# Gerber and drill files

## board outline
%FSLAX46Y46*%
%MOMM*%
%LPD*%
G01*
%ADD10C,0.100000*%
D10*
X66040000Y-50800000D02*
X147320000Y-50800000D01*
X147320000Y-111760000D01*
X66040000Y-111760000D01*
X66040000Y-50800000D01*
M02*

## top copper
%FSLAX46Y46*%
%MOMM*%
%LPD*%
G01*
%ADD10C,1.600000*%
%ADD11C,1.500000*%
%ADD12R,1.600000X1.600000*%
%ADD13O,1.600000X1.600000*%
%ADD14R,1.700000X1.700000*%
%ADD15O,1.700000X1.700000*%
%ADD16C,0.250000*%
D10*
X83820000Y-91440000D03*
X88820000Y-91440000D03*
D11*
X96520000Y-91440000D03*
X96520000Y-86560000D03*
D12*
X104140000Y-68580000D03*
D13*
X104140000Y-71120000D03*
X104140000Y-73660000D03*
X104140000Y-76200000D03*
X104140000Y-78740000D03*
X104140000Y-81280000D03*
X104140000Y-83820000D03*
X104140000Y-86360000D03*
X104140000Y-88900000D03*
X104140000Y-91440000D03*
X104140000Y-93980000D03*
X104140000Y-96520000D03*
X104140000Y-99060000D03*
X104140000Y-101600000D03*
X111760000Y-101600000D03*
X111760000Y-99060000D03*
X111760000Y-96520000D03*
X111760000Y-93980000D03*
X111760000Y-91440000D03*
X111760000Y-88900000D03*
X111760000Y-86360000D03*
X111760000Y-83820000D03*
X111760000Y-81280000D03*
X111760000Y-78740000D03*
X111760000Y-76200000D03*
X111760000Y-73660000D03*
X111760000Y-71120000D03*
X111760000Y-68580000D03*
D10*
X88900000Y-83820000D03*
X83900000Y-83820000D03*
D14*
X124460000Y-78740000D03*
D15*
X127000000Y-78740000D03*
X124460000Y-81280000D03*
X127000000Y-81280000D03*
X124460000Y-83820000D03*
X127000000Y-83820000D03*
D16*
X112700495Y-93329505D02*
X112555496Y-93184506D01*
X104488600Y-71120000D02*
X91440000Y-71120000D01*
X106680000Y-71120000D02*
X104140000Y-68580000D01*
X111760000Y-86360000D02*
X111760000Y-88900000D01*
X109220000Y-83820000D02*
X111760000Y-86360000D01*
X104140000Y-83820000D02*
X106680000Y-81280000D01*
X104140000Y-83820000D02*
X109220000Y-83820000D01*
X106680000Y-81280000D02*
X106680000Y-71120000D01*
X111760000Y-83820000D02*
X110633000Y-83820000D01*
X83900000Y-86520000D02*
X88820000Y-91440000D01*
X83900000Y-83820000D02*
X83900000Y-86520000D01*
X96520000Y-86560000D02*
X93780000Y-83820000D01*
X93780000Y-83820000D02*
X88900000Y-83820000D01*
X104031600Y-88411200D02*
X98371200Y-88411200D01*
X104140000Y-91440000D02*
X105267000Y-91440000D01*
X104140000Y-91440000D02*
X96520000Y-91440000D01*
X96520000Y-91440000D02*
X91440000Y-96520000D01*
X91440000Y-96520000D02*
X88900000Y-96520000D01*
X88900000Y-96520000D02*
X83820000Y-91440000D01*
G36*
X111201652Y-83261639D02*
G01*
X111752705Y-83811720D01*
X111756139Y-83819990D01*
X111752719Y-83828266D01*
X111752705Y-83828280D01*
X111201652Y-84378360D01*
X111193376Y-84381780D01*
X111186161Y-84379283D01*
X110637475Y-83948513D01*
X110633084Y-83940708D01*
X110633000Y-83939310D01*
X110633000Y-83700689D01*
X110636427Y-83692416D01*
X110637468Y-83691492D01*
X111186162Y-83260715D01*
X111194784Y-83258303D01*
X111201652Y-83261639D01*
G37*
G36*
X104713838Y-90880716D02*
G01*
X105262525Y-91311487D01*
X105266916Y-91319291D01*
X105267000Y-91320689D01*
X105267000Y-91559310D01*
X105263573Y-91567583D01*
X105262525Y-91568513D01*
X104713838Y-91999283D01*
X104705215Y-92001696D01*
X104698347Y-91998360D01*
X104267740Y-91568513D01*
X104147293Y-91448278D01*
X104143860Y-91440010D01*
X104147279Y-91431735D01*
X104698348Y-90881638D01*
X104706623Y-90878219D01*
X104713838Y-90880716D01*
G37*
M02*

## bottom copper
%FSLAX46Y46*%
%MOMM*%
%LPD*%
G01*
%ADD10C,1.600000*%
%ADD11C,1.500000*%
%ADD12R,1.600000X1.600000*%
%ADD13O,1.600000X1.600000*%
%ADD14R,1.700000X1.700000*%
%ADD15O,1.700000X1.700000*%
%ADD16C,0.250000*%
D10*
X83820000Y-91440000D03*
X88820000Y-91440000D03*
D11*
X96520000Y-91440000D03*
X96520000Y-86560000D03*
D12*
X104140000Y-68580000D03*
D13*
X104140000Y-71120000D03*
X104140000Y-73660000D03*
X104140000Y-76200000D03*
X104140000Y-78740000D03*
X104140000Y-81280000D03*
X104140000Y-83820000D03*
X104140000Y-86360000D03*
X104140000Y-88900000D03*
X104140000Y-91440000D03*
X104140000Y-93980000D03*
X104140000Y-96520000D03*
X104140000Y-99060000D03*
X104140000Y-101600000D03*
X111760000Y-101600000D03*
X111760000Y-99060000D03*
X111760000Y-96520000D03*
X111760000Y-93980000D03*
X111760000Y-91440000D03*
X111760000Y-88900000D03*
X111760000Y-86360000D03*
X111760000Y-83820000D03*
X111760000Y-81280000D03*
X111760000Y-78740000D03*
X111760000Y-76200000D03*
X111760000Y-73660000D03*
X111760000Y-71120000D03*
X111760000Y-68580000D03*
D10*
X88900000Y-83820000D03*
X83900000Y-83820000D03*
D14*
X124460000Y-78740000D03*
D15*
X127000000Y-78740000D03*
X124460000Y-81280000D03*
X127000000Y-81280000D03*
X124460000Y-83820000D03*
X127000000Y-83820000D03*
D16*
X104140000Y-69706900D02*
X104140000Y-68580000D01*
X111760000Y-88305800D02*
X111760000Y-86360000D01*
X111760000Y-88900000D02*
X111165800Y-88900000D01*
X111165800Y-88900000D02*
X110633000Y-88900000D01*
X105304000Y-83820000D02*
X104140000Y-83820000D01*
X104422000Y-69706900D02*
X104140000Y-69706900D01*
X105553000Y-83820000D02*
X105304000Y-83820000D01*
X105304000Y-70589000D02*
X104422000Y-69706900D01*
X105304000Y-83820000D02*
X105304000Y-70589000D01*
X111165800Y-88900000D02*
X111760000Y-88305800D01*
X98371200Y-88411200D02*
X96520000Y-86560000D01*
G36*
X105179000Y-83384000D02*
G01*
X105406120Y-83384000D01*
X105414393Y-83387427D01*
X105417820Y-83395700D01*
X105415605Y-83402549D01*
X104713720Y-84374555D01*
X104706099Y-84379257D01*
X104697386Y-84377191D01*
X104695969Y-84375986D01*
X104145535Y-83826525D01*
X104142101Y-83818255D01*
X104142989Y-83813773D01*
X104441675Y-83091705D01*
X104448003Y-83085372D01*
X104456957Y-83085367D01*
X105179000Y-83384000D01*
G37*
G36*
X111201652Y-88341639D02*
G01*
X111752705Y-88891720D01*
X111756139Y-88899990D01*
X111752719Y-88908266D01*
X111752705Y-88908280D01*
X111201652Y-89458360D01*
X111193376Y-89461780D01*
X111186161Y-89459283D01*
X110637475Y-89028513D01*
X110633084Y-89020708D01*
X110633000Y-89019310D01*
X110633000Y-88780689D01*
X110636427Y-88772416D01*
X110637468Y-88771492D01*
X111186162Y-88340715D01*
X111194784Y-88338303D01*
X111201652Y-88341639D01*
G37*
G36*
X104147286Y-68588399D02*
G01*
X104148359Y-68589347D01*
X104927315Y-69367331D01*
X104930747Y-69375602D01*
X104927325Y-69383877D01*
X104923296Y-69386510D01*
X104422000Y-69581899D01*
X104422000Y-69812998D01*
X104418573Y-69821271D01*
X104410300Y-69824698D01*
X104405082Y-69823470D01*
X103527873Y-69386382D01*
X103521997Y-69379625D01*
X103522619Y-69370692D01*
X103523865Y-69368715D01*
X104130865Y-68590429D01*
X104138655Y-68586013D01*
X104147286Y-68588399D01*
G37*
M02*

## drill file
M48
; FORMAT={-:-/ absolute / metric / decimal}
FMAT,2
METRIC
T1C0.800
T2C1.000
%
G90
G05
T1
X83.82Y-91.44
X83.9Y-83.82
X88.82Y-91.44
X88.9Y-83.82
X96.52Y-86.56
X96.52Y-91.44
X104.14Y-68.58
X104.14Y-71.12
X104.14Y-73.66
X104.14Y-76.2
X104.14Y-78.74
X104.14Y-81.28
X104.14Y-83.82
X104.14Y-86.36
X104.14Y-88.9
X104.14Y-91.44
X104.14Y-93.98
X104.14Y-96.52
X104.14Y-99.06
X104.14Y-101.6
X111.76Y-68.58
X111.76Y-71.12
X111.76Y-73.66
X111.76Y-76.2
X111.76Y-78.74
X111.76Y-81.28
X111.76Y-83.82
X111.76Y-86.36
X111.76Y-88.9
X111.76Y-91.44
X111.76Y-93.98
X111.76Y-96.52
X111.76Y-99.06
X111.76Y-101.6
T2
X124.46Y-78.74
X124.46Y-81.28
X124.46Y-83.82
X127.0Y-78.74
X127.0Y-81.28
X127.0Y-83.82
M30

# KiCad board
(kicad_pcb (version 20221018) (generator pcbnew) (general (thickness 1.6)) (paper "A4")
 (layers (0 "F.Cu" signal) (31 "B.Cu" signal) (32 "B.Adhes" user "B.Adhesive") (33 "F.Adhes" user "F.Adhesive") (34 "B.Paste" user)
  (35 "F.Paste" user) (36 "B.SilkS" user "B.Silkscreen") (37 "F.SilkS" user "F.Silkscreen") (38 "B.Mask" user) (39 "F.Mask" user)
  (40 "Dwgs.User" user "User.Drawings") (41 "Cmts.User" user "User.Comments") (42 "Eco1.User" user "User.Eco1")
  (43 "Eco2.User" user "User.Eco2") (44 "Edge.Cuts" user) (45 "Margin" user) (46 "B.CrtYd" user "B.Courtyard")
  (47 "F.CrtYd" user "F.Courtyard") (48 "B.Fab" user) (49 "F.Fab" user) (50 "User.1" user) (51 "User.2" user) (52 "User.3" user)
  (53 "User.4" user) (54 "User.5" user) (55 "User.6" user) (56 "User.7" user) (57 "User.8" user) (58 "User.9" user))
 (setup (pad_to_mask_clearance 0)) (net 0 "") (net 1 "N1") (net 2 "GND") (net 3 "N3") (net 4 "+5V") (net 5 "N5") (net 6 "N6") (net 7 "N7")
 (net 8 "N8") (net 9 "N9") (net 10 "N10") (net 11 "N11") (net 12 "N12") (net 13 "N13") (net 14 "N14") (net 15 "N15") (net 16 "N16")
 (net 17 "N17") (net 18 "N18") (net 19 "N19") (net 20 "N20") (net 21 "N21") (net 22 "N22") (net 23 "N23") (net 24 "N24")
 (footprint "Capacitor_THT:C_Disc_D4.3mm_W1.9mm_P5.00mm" (layer "F.Cu") (at 83.82 91.44)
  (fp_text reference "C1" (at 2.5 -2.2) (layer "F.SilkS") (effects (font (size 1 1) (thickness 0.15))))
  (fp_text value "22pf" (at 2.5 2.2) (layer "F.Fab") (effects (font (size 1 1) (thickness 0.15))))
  (pad "1" thru_hole circle (at 0 0) (size 1.6 1.6) (drill 0.8) (layers "*.Cu" "*.Mask") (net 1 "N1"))
  (pad "2" thru_hole circle (at 5 0) (size 1.6 1.6) (drill 0.8) (layers "*.Cu" "*.Mask") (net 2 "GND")))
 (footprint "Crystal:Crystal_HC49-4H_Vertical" (layer "F.Cu") (at 96.52 91.44 90)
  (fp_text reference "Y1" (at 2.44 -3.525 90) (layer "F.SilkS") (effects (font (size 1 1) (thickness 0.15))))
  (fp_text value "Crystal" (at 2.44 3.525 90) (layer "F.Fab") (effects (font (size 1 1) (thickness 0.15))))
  (pad "1" thru_hole circle (at 0 0 90) (size 1.5 1.5) (drill 0.8) (layers "*.Cu" "*.Mask") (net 1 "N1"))
  (pad "2" thru_hole circle (at 4.88 0 90) (size 1.5 1.5) (drill 0.8) (layers "*.Cu" "*.Mask") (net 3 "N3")))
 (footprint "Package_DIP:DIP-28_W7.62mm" (layer "F.Cu") (at 104.14 68.58)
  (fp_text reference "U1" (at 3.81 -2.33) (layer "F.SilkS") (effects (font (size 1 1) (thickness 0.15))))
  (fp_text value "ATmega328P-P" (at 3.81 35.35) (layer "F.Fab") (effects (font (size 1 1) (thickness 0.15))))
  (pad "1" thru_hole rect (at 0 0) (size 1.6 1.6) (drill 0.8) (layers "*.Cu" "*.Mask") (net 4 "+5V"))
  (pad "2" thru_hole oval (at 0 2.54) (size 1.6 1.6) (drill 0.8) (layers "*.Cu" "*.Mask") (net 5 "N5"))
  (pad "3" thru_hole oval (at 0 5.08) (size 1.6 1.6) (drill 0.8) (layers "*.Cu" "*.Mask") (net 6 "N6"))
  (pad "4" thru_hole oval (at 0 7.62) (size 1.6 1.6) (drill 0.8) (layers "*.Cu" "*.Mask") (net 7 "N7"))
  (pad "5" thru_hole oval (at 0 10.16) (size 1.6 1.6) (drill 0.8) (layers "*.Cu" "*.Mask") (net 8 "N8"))
  (pad "6" thru_hole oval (at 0 12.7) (size 1.6 1.6) (drill 0.8) (layers "*.Cu" "*.Mask") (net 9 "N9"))
  (pad "7" thru_hole oval (at 0 15.24) (size 1.6 1.6) (drill 0.8) (layers "*.Cu" "*.Mask") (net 4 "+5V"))
  (pad "8" thru_hole oval (at 0 17.78) (size 1.6 1.6) (drill 0.8) (layers "*.Cu" "*.Mask") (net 2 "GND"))
  (pad "9" thru_hole oval (at 0 20.32) (size 1.6 1.6) (drill 0.8) (layers "*.Cu" "*.Mask") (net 3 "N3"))
  (pad "10" thru_hole oval (at 0 22.86) (size 1.6 1.6) (drill 0.8) (layers "*.Cu" "*.Mask") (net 1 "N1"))
  (pad "11" thru_hole oval (at 0 25.4) (size 1.6 1.6) (drill 0.8) (layers "*.Cu" "*.Mask") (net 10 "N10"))
  (pad "12" thru_hole oval (at 0 27.94) (size 1.6 1.6) (drill 0.8) (layers "*.Cu" "*.Mask") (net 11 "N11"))
  (pad "13" thru_hole oval (at 0 30.48) (size 1.6 1.6) (drill 0.8) (layers "*.Cu" "*.Mask") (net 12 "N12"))
  (pad "14" thru_hole oval (at 0 33.02) (size 1.6 1.6) (drill 0.8) (layers "*.Cu" "*.Mask") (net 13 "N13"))
  (pad "15" thru_hole oval (at 7.62 33.02) (size 1.6 1.6) (drill 0.8) (layers "*.Cu" "*.Mask") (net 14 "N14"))
  (pad "16" thru_hole oval (at 7.62 30.48) (size 1.6 1.6) (drill 0.8) (layers "*.Cu" "*.Mask") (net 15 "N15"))
  (pad "17" thru_hole oval (at 7.62 27.94) (size 1.6 1.6) (drill 0.8) (layers "*.Cu" "*.Mask") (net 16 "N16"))
  (pad "18" thru_hole oval (at 7.62 25.4) (size 1.6 1.6) (drill 0.8) (layers "*.Cu" "*.Mask") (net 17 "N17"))
  (pad "19" thru_hole oval (at 7.62 22.86) (size 1.6 1.6) (drill 0.8) (layers "*.Cu" "*.Mask") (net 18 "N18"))
  (pad "20" thru_hole oval (at 7.62 20.32) (size 1.6 1.6) (drill 0.8) (layers "*.Cu" "*.Mask") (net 4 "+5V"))
  (pad "21" thru_hole oval (at 7.62 17.78) (size 1.6 1.6) (drill 0.8) (layers "*.Cu" "*.Mask") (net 4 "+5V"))
  (pad "22" thru_hole oval (at 7.62 15.24) (size 1.6 1.6) (drill 0.8) (layers "*.Cu" "*.Mask") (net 2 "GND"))
  (pad "23" thru_hole oval (at 7.62 12.7) (size 1.6 1.6) (drill 0.8) (layers "*.Cu" "*.Mask") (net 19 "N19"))
  (pad "24" thru_hole oval (at 7.62 10.16) (size 1.6 1.6) (drill 0.8) (layers "*.Cu" "*.Mask") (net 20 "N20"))
  (pad "25" thru_hole oval (at 7.62 7.62) (size 1.6 1.6) (drill 0.8) (layers "*.Cu" "*.Mask") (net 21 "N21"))
  (pad "26" thru_hole oval (at 7.62 5.08) (size 1.6 1.6) (drill 0.8) (layers "*.Cu" "*.Mask") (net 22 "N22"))
  (pad "27" thru_hole oval (at 7.62 2.54) (size 1.6 1.6) (drill 0.8) (layers "*.Cu" "*.Mask") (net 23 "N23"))
  (pad "28" thru_hole oval (at 7.62 0) (size 1.6 1.6) (drill 0.8) (layers "*.Cu" "*.Mask") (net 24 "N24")))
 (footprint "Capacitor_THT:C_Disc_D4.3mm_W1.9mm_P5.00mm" (layer "F.Cu") (at 88.9 83.82 180)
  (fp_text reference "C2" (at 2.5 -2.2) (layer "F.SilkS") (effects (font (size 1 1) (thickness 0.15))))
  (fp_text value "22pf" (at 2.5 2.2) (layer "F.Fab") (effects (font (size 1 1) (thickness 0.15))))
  (pad "1" thru_hole circle (at 0 0 180) (size 1.6 1.6) (drill 0.8) (layers "*.Cu" "*.Mask") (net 3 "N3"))
  (pad "2" thru_hole circle (at 5 0 180) (size 1.6 1.6) (drill 0.8) (layers "*.Cu" "*.Mask") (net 2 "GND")))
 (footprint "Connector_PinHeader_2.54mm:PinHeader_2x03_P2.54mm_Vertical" (layer "F.Cu") (at 124.46 78.74)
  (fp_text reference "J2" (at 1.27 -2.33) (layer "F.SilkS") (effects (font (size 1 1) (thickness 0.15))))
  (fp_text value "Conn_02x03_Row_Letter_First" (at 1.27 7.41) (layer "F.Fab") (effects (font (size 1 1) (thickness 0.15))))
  (pad "1" thru_hole rect (at 0 0) (size 1.7 1.7) (drill 1) (layers "*.Cu" "*.Mask"))
  (pad "2" thru_hole oval (at 2.54 0) (size 1.7 1.7) (drill 1) (layers "*.Cu" "*.Mask"))
  (pad "3" thru_hole oval (at 0 2.54) (size 1.7 1.7) (drill 1) (layers "*.Cu" "*.Mask"))
  (pad "4" thru_hole oval (at 2.54 2.54) (size 1.7 1.7) (drill 1) (layers "*.Cu" "*.Mask"))
  (pad "5" thru_hole oval (at 0 5.08) (size 1.7 1.7) (drill 1) (layers "*.Cu" "*.Mask"))
  (pad "6" thru_hole oval (at 2.54 5.08) (size 1.7 1.7) (drill 1) (layers "*.Cu" "*.Mask")))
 (gr_rect (start 66.04 50.8) (end 147.32 111.76) (stroke (width 0.1) (type default)) (fill none) (layer "Edge.Cuts"))
 (segment (start 112.700495 93.329505) (end 112.555496 93.184506) (width 0.25) (layer "F.Cu") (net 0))
 (segment (start 104.4886 71.12) (end 91.44 71.12) (width 0.25) (layer "F.Cu") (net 5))
 (segment (start 106.68 71.12) (end 104.14 68.58) (width 0.25) (layer "F.Cu") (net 4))
 (segment (start 111.76 86.36) (end 111.76 88.9) (width 0.25) (layer "F.Cu") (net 4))
 (segment (start 109.22 83.82) (end 111.76 86.36) (width 0.25) (layer "F.Cu") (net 4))
 (segment (start 104.14 83.82) (end 106.68 81.28) (width 0.25) (layer "F.Cu") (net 4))
 (segment (start 104.14 83.82) (end 109.22 83.82) (width 0.25) (layer "F.Cu") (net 4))
 (segment (start 106.68 81.28) (end 106.68 71.12) (width 0.25) (layer "F.Cu") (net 4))
 (segment (start 104.14 69.7069) (end 104.14 68.58) (width 0.25) (layer "B.Cu") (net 4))
 (segment (start 111.76 88.3058) (end 111.76 86.36) (width 0.25) (layer "B.Cu") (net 4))
 (segment (start 111.76 88.9) (end 111.1658 88.9) (width 0.25) (layer "B.Cu") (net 4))
 (segment (start 111.1658 88.9) (end 110.633 88.9) (width 0.25) (layer "B.Cu") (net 4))
 (segment (start 105.304 83.82) (end 104.14 83.82) (width 0.25) (layer "B.Cu") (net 4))
 (segment (start 104.422 69.7069) (end 104.14 69.7069) (width 0.25) (layer "B.Cu") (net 4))
 (segment (start 105.553 83.82) (end 105.304 83.82) (width 0.25) (layer "B.Cu") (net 4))
 (segment (start 105.304 70.589) (end 104.422 69.7069) (width 0.25) (layer "B.Cu") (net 4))
 (segment (start 105.304 83.82) (end 105.304 70.589) (width 0.25) (layer "B.Cu") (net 4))
 (segment (start 111.1658 88.9) (end 111.76 88.3058) (width 0.25) (layer "B.Cu") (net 4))
 (segment (start 111.76 83.82) (end 110.633 83.82) (width 0.25) (layer "F.Cu") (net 2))
 (segment (start 83.9 86.52) (end 88.82 91.44) (width 0.25) (layer "F.Cu") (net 2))
 (segment (start 83.9 83.82) (end 83.9 86.52) (width 0.25) (layer "F.Cu") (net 2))
 (segment (start 96.52 86.56) (end 93.78 83.82) (width 0.25) (layer "F.Cu") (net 3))
 (segment (start 93.78 83.82) (end 88.9 83.82) (width 0.25) (layer "F.Cu") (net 3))
 (segment (start 104.0316 88.4112) (end 98.3712 88.4112) (width 0.25) (layer "F.Cu") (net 3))
 (segment (start 98.3712 88.4112) (end 96.52 86.56) (width 0.25) (layer "B.Cu") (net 3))
 (segment (start 104.14 91.44) (end 105.267 91.44) (width 0.25) (layer "F.Cu") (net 1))
 (segment (start 104.14 91.44) (end 96.52 91.44) (width 0.25) (layer "F.Cu") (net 1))
 (segment (start 96.52 91.44) (end 91.44 96.52) (width 0.25) (layer "F.Cu") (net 1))
 (segment (start 91.44 96.52) (end 88.9 96.52) (width 0.25) (layer "F.Cu") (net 1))
 (segment (start 88.9 96.52) (end 83.82 91.44) (width 0.25) (layer "F.Cu") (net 1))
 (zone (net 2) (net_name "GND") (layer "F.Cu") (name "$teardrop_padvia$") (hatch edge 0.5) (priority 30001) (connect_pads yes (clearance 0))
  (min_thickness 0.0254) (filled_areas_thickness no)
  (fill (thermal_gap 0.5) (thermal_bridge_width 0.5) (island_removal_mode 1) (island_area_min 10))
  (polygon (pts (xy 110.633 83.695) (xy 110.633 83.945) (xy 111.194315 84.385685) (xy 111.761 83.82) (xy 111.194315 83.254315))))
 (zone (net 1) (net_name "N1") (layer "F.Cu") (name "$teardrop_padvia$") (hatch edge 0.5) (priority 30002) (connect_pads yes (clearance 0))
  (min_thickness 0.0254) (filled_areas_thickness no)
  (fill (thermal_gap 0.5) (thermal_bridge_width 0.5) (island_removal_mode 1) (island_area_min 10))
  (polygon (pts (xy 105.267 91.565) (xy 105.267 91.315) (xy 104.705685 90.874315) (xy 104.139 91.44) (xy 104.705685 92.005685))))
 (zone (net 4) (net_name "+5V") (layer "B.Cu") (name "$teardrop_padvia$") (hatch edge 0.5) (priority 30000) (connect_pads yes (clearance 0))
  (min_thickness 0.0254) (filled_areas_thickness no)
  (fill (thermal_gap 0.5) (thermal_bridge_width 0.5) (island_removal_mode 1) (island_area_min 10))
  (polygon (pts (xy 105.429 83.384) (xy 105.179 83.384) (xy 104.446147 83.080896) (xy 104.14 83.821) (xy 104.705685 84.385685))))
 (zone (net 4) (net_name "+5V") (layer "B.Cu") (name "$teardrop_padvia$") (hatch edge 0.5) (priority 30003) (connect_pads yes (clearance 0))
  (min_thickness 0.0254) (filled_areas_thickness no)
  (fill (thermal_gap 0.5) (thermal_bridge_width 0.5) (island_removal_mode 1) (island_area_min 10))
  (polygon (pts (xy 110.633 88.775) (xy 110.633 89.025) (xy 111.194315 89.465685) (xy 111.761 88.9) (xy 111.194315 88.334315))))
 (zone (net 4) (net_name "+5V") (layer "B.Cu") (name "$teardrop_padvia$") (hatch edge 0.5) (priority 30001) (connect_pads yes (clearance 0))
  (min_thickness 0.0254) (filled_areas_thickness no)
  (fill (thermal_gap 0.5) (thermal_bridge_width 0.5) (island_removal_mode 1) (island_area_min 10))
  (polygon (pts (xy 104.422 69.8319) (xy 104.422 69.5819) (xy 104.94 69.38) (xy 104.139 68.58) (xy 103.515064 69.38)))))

